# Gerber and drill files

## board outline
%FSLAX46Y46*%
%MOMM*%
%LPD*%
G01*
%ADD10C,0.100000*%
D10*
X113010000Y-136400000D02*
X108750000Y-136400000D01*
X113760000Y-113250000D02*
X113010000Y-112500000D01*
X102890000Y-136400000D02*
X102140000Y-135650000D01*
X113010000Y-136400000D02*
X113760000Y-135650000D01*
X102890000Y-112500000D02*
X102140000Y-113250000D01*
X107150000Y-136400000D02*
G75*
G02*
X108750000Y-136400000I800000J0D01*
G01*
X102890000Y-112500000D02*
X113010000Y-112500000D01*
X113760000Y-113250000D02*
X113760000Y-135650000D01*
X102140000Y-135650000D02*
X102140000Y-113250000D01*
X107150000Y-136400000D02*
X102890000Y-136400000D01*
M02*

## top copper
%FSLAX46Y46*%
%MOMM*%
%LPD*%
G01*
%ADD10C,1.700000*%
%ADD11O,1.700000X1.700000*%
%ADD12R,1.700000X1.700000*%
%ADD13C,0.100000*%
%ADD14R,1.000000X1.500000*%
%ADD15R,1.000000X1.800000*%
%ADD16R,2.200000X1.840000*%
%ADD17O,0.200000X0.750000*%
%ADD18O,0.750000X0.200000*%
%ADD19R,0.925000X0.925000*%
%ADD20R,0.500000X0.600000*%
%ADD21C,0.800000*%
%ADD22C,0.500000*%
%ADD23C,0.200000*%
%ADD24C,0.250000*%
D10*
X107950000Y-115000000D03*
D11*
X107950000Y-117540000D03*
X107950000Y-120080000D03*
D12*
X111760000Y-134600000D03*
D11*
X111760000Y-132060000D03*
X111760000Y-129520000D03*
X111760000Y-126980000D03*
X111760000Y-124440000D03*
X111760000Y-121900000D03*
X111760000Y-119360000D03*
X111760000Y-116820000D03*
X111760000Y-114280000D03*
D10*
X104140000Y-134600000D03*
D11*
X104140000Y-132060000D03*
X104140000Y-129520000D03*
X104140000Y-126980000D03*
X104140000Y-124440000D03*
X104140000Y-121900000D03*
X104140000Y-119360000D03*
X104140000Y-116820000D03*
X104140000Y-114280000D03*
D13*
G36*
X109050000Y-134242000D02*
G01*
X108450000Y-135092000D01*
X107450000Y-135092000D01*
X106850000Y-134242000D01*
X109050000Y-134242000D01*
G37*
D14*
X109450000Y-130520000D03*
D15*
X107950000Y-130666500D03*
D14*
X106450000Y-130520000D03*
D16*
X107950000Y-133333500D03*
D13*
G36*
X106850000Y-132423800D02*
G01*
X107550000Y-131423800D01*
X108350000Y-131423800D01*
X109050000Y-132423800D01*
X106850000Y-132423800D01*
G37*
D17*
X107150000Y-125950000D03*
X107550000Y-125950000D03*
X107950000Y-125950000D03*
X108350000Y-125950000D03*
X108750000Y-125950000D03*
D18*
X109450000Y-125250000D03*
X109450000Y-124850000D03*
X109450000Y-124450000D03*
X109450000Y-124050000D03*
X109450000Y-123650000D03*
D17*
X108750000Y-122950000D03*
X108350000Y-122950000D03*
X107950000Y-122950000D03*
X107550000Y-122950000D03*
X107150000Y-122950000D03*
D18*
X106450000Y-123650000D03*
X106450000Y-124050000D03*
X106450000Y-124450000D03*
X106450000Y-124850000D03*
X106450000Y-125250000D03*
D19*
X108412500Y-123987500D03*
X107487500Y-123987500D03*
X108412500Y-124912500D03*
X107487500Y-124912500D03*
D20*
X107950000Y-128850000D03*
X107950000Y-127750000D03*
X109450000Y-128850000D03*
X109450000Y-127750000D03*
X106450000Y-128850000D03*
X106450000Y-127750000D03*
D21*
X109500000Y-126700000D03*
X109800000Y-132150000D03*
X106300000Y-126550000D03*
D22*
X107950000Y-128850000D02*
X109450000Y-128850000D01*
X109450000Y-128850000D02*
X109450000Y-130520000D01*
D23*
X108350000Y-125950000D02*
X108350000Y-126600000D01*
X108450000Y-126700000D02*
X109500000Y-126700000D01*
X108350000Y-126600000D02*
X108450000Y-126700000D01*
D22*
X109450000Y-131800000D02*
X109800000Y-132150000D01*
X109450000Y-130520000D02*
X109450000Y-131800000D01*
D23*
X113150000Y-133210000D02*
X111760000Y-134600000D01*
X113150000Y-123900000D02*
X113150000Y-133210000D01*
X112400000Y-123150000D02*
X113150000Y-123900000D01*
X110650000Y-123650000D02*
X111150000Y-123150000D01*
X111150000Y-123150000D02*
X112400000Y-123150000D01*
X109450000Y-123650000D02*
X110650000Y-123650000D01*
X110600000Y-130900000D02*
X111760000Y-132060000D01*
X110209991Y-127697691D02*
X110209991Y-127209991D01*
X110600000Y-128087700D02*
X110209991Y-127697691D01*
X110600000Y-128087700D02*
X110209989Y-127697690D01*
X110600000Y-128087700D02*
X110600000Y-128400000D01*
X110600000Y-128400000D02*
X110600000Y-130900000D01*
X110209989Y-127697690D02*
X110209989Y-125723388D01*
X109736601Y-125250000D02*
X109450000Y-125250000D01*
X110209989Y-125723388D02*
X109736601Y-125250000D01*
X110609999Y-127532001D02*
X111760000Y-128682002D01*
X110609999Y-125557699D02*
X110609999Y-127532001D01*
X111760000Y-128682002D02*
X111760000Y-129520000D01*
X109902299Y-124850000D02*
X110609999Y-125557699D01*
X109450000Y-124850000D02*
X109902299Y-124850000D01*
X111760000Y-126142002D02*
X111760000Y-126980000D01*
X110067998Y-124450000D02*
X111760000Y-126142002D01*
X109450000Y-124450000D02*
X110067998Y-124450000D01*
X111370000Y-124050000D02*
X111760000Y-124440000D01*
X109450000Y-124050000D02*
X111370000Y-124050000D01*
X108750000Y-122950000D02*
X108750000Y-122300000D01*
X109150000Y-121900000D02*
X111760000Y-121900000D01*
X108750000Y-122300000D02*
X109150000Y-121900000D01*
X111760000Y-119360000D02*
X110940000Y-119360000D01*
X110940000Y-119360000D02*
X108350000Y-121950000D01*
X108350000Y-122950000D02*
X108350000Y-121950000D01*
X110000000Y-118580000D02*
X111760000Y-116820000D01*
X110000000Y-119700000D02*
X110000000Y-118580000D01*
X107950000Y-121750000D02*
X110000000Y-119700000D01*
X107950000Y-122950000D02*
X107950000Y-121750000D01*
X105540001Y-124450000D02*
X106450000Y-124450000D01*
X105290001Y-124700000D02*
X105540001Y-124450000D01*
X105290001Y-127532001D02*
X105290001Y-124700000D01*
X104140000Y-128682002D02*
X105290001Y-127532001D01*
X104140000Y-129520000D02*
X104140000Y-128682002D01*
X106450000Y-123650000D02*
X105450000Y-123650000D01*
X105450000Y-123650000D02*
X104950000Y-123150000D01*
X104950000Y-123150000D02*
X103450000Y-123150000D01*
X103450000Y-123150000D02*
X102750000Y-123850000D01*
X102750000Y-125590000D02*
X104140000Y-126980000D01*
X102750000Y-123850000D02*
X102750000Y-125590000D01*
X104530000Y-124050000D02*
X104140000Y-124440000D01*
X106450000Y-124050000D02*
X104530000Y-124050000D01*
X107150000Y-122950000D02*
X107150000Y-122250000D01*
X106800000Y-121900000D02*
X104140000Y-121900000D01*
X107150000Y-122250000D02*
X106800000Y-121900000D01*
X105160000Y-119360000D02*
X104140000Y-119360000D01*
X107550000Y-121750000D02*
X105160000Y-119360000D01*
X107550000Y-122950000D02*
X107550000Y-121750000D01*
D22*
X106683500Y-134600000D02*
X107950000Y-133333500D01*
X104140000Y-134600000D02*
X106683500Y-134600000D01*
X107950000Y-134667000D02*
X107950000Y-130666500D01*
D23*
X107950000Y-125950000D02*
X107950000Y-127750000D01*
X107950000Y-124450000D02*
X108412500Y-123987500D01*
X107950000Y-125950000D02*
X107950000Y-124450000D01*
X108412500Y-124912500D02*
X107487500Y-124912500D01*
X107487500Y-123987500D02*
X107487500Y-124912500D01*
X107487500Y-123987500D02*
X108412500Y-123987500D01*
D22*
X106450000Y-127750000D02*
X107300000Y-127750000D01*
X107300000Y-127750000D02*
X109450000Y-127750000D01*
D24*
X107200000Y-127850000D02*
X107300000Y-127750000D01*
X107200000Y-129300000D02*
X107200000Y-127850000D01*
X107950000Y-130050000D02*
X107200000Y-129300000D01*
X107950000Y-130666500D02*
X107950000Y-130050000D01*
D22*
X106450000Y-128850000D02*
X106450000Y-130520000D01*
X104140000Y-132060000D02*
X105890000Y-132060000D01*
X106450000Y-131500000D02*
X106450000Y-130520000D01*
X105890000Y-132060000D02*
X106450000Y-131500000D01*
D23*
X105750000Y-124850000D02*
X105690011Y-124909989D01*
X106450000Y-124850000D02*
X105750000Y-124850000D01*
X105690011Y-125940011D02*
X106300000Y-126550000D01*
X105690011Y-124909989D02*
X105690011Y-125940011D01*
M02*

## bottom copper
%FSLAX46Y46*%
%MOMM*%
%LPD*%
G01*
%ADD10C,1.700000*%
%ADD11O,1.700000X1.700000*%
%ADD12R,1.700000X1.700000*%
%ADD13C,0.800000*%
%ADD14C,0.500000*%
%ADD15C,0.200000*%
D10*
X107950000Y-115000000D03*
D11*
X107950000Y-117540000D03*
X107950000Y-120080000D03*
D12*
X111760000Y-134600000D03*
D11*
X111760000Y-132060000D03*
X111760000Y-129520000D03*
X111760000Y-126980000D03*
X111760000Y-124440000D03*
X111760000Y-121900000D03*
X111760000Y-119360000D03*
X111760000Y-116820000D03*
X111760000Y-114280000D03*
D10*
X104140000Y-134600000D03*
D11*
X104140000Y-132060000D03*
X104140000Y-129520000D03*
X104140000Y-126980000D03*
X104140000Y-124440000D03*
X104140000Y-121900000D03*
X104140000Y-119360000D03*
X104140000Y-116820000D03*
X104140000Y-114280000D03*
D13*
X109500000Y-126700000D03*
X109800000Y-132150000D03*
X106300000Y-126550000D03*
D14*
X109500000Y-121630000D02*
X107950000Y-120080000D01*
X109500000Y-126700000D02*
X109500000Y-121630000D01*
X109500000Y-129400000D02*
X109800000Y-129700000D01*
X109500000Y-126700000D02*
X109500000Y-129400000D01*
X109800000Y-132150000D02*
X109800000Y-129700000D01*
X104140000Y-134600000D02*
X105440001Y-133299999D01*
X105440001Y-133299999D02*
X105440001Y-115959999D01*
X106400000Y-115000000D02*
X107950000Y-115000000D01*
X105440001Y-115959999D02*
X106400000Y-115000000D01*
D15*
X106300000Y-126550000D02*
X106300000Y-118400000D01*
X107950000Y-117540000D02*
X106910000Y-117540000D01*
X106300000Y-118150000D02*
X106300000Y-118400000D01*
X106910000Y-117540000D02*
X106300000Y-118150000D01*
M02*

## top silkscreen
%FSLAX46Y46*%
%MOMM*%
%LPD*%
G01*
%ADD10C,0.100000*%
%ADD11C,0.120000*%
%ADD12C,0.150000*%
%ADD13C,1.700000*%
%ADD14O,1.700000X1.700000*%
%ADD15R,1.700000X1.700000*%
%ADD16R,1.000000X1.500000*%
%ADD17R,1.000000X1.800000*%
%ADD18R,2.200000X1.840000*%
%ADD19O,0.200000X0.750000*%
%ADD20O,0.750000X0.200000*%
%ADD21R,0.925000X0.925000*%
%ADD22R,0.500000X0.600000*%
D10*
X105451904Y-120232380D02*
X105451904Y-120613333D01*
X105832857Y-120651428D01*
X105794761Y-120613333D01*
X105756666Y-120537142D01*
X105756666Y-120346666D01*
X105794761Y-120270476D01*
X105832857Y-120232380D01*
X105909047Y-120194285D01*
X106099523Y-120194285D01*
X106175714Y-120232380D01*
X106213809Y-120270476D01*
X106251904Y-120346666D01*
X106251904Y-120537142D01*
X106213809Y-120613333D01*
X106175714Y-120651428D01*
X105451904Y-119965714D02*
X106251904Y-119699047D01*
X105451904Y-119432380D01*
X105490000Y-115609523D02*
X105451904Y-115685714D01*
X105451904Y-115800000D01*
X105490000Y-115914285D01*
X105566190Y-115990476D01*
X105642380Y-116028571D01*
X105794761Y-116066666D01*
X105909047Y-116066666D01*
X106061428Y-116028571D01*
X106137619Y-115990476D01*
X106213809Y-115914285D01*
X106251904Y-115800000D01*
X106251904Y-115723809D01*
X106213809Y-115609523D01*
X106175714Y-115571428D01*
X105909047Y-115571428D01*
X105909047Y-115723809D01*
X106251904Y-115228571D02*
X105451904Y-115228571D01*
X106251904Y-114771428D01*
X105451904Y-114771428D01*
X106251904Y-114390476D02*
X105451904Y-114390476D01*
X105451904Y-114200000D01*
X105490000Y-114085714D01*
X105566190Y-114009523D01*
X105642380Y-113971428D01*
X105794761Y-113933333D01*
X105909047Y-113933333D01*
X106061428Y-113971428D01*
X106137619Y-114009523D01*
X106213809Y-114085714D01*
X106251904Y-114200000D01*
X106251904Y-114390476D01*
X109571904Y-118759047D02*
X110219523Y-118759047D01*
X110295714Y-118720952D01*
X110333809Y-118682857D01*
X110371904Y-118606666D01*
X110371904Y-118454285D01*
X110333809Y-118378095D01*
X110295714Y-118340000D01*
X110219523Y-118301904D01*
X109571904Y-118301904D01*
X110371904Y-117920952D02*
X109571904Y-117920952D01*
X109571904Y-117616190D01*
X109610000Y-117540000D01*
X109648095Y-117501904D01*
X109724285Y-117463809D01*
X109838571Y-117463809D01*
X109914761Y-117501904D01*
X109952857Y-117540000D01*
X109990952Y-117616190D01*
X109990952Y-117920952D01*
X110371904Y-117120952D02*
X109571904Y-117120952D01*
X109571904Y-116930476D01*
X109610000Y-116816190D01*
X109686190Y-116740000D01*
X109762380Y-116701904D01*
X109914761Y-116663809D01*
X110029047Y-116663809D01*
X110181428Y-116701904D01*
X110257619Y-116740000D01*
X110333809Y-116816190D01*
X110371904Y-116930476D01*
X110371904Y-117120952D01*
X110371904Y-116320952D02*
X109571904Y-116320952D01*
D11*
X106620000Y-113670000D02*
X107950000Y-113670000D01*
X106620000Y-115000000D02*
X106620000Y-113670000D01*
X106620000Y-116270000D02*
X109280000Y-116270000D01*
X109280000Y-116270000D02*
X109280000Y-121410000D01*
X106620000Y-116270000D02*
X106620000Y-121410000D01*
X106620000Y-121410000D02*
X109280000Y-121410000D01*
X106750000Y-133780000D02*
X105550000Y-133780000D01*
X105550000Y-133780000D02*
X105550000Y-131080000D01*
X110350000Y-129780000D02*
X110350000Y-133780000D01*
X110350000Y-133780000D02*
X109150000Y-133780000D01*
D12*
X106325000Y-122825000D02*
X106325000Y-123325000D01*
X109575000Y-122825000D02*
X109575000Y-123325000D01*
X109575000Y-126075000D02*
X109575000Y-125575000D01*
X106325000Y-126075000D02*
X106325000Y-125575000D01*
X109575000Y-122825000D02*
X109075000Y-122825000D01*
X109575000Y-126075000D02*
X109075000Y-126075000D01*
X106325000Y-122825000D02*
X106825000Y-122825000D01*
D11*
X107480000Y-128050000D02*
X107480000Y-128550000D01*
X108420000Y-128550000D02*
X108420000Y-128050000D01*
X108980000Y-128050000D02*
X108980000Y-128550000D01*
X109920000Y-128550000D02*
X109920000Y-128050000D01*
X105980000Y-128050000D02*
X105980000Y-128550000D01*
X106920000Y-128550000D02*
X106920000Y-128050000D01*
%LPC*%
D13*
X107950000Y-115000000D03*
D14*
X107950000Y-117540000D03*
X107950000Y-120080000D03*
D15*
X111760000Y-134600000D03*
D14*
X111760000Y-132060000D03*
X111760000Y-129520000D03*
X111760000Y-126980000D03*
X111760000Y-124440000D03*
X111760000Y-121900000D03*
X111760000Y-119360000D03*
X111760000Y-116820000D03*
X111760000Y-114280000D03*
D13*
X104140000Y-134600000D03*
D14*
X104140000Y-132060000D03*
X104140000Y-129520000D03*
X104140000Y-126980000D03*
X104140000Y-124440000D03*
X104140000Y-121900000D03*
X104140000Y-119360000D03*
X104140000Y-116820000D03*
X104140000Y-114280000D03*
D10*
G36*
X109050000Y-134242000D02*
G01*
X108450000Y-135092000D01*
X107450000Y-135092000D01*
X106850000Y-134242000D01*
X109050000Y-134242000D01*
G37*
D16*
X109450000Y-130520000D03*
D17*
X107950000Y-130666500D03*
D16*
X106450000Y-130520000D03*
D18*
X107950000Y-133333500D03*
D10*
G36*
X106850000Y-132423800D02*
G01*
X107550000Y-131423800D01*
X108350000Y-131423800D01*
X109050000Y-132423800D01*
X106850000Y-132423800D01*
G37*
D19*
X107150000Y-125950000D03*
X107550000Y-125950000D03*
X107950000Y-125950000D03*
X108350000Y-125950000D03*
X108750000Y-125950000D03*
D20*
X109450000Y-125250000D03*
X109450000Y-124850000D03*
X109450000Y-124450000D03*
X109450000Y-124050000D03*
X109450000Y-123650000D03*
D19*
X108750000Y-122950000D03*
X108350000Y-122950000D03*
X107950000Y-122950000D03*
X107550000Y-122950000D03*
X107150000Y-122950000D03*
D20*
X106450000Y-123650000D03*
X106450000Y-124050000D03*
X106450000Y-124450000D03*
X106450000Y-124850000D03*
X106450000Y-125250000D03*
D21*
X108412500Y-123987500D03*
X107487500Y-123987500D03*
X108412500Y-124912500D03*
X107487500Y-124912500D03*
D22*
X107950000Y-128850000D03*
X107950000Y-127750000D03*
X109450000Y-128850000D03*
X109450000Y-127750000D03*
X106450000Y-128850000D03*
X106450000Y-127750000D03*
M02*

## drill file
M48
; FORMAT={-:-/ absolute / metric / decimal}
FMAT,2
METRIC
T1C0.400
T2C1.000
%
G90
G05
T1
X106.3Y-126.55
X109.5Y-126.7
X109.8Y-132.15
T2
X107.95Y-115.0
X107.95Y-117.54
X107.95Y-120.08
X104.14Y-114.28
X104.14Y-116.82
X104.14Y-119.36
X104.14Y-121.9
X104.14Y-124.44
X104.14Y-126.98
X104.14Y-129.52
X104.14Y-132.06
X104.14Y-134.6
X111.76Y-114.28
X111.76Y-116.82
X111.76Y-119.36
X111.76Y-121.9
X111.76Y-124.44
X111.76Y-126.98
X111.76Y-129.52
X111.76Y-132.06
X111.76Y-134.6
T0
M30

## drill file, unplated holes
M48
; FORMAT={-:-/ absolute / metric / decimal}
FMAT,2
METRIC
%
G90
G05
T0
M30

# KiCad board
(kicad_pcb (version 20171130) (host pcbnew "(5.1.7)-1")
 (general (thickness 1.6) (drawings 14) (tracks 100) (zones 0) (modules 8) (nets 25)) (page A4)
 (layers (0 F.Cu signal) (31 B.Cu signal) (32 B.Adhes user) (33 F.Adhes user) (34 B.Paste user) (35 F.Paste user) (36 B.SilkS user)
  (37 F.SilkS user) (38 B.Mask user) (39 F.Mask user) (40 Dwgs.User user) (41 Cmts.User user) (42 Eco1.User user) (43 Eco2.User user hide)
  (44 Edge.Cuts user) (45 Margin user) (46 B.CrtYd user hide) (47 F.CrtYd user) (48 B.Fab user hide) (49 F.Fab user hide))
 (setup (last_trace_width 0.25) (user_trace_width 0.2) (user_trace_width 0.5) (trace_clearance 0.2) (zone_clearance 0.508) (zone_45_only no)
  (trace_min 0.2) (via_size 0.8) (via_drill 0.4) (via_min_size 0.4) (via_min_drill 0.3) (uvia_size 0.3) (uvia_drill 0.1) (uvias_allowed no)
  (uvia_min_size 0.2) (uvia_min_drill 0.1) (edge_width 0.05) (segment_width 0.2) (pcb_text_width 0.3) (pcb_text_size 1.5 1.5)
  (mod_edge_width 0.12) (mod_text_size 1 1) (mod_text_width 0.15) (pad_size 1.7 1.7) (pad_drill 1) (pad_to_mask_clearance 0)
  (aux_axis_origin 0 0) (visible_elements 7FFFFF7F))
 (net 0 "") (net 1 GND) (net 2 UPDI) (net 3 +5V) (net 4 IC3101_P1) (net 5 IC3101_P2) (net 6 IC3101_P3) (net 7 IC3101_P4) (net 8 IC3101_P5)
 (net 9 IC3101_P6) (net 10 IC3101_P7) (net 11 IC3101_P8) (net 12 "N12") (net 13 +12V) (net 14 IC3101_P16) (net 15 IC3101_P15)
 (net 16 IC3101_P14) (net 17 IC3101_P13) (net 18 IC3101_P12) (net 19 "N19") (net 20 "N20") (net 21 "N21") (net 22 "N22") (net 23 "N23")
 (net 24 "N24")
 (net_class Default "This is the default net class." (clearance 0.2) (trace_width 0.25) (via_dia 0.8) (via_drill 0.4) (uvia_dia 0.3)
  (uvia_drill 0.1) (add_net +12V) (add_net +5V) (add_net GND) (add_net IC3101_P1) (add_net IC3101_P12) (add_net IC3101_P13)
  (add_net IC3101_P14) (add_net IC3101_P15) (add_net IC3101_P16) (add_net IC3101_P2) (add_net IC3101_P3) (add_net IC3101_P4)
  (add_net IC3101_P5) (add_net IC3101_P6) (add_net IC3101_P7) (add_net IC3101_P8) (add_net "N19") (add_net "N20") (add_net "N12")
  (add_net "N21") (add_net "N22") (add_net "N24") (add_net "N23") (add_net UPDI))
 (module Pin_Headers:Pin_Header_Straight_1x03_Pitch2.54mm (layer F.Cu) (at 107.95 115)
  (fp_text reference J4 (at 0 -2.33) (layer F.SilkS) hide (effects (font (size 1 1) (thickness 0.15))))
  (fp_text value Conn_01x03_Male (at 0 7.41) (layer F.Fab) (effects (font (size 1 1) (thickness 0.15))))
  (fp_line (start -1.33 -1.33) (end 0 -1.33) (layer F.SilkS) (width 0.12))
  (fp_line (start -1.33 0) (end -1.33 -1.33) (layer F.SilkS) (width 0.12))
  (fp_line (start -1.33 1.27) (end 1.33 1.27) (layer F.SilkS) (width 0.12))
  (fp_line (start 1.33 1.27) (end 1.33 6.41) (layer F.SilkS) (width 0.12))
  (fp_line (start -1.33 1.27) (end -1.33 6.41) (layer F.SilkS) (width 0.12))
  (fp_line (start -1.33 6.41) (end 1.33 6.41) (layer F.SilkS) (width 0.12))
  (pad 1 thru_hole circle (at 0 0) (size 1.7 1.7) (drill 1) (layers *.Cu *.Mask) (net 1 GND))
  (pad 2 thru_hole oval (at 0 2.54) (size 1.7 1.7) (drill 1) (layers *.Cu *.Mask) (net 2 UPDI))
  (pad 3 thru_hole oval (at 0 5.08) (size 1.7 1.7) (drill 1) (layers *.Cu *.Mask) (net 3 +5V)))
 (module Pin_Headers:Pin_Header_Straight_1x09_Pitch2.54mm (layer B.Cu) (at 111.76 134.6)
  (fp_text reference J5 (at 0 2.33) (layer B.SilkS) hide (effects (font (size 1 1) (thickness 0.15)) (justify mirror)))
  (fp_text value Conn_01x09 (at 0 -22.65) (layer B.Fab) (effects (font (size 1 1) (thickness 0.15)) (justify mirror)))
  (pad 1 thru_hole rect (at 0 0) (size 1.7 1.7) (drill 1) (layers *.Cu *.Mask) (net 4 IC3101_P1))
  (pad 2 thru_hole oval (at 0 -2.54) (size 1.7 1.7) (drill 1) (layers *.Cu *.Mask) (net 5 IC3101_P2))
  (pad 3 thru_hole oval (at 0 -5.08) (size 1.7 1.7) (drill 1) (layers *.Cu *.Mask) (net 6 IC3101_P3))
  (pad 4 thru_hole oval (at 0 -7.62) (size 1.7 1.7) (drill 1) (layers *.Cu *.Mask) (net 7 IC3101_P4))
  (pad 5 thru_hole oval (at 0 -10.16) (size 1.7 1.7) (drill 1) (layers *.Cu *.Mask) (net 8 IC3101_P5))
  (pad 6 thru_hole oval (at 0 -12.7) (size 1.7 1.7) (drill 1) (layers *.Cu *.Mask) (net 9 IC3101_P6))
  (pad 7 thru_hole oval (at 0 -15.24) (size 1.7 1.7) (drill 1) (layers *.Cu *.Mask) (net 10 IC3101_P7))
  (pad 8 thru_hole oval (at 0 -17.78) (size 1.7 1.7) (drill 1) (layers *.Cu *.Mask) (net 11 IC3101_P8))
  (pad 9 thru_hole oval (at 0 -20.32) (size 1.7 1.7) (drill 1) (layers *.Cu *.Mask) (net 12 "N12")))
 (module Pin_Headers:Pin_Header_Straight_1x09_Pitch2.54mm (layer B.Cu) (at 104.14 134.6)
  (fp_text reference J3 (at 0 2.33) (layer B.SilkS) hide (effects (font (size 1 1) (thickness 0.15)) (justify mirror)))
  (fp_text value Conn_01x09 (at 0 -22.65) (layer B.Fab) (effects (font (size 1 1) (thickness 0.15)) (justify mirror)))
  (pad 1 thru_hole circle (at 0 0) (size 1.7 1.7) (drill 1) (layers *.Cu *.Mask) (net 1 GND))
  (pad 2 thru_hole oval (at 0 -2.54) (size 1.7 1.7) (drill 1) (layers *.Cu *.Mask) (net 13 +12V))
  (pad 3 thru_hole oval (at 0 -5.08) (size 1.7 1.7) (drill 1) (layers *.Cu *.Mask) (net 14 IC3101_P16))
  (pad 4 thru_hole oval (at 0 -7.62) (size 1.7 1.7) (drill 1) (layers *.Cu *.Mask) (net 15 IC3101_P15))
  (pad 5 thru_hole oval (at 0 -10.16) (size 1.7 1.7) (drill 1) (layers *.Cu *.Mask) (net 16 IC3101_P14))
  (pad 6 thru_hole oval (at 0 -12.7) (size 1.7 1.7) (drill 1) (layers *.Cu *.Mask) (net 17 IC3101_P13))
  (pad 7 thru_hole oval (at 0 -15.24) (size 1.7 1.7) (drill 1) (layers *.Cu *.Mask) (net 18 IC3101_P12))
  (pad 8 thru_hole oval (at 0 -17.78) (size 1.7 1.7) (drill 1) (layers *.Cu *.Mask) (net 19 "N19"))
  (pad 9 thru_hole oval (at 0 -20.32) (size 1.7 1.7) (drill 1) (layers *.Cu *.Mask) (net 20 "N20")))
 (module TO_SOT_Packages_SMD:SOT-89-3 (layer F.Cu) (at 107.95 132 270)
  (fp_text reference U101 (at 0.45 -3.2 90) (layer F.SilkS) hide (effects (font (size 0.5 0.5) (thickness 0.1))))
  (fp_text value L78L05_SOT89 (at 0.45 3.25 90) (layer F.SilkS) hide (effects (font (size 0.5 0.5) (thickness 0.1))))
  (fp_line (start 1.78 1.2) (end 1.78 2.4) (layer F.SilkS) (width 0.12))
  (fp_line (start 1.78 2.4) (end -0.92 2.4) (layer F.SilkS) (width 0.12))
  (fp_line (start -2.22 -2.4) (end 1.78 -2.4) (layer F.SilkS) (width 0.12))
  (fp_line (start 1.78 -2.4) (end 1.78 -1.2) (layer F.SilkS) (width 0.12))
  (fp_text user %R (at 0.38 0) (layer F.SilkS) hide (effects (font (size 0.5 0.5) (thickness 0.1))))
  (pad 2 smd trapezoid (at 2.667 0 180) (size 1.6 0.85) (rect_delta 0 0.6) (layers F.Cu F.Paste F.Mask) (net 1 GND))
  (pad 1 smd rect (at -1.48 -1.5 180) (size 1 1.5) (layers F.Cu F.Paste F.Mask) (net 3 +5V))
  (pad 2 smd rect (at -1.3335 0 180) (size 1 1.8) (layers F.Cu F.Paste F.Mask) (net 1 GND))
  (pad 3 smd rect (at -1.48 1.5 180) (size 1 1.5) (layers F.Cu F.Paste F.Mask) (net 13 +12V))
  (pad 2 smd rect (at 1.3335 0 180) (size 2.2 1.84) (layers F.Cu F.Paste F.Mask) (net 1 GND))
  (pad 2 smd trapezoid (at -0.0762 0) (size 1.5 1) (rect_delta 0 0.7) (layers F.Cu F.Paste F.Mask) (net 1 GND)))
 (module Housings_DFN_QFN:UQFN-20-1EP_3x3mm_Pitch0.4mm (layer F.Cu) (at 107.95 124.45 90)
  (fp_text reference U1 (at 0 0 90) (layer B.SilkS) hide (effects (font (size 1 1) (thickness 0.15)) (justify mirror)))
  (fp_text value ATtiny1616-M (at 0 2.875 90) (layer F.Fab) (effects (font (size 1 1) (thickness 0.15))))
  (fp_line (start 1.625 -1.625) (end 1.125 -1.625) (layer F.SilkS) (width 0.15))
  (fp_line (start 1.625 1.625) (end 1.125 1.625) (layer F.SilkS) (width 0.15))
  (fp_line (start -1.625 1.625) (end -1.125 1.625) (layer F.SilkS) (width 0.15))
  (fp_line (start -1.625 -1.625) (end -1.125 -1.625) (layer F.SilkS) (width 0.15))
  (fp_line (start 1.625 1.625) (end 1.625 1.125) (layer F.SilkS) (width 0.15))
  (fp_line (start -1.625 1.625) (end -1.625 1.125) (layer F.SilkS) (width 0.15))
  (fp_line (start 1.625 -1.625) (end 1.625 -1.125) (layer F.SilkS) (width 0.15))
  (pad 1 smd oval (at -1.5 -0.8 90) (size 0.75 0.2) (layers F.Cu F.Paste F.Mask) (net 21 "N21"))
  (pad 2 smd oval (at -1.5 -0.4 90) (size 0.75 0.2) (layers F.Cu F.Paste F.Mask) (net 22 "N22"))
  (pad 3 smd oval (at -1.5 0 90) (size 0.75 0.2) (layers F.Cu F.Paste F.Mask) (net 1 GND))
  (pad 4 smd oval (at -1.5 0.4 90) (size 0.75 0.2) (layers F.Cu F.Paste F.Mask) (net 3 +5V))
  (pad 5 smd oval (at -1.5 0.8 90) (size 0.75 0.2) (layers F.Cu F.Paste F.Mask) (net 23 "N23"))
  (pad 6 smd oval (at -0.8 1.5 180) (size 0.75 0.2) (layers F.Cu F.Paste F.Mask) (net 5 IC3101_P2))
  (pad 7 smd oval (at -0.4 1.5 180) (size 0.75 0.2) (layers F.Cu F.Paste F.Mask) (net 6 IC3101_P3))
  (pad 8 smd oval (at 0 1.5 180) (size 0.75 0.2) (layers F.Cu F.Paste F.Mask) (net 7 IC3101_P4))
  (pad 9 smd oval (at 0.4 1.5 180) (size 0.75 0.2) (layers F.Cu F.Paste F.Mask) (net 8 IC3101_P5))
  (pad 10 smd oval (at 0.8 1.5 180) (size 0.75 0.2) (layers F.Cu F.Paste F.Mask) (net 4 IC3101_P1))
  (pad 11 smd oval (at 1.5 0.8 90) (size 0.75 0.2) (layers F.Cu F.Paste F.Mask) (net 9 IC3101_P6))
  (pad 12 smd oval (at 1.5 0.4 90) (size 0.75 0.2) (layers F.Cu F.Paste F.Mask) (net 10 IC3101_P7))
  (pad 13 smd oval (at 1.5 0 90) (size 0.75 0.2) (layers F.Cu F.Paste F.Mask) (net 11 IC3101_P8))
  (pad 14 smd oval (at 1.5 -0.4 90) (size 0.75 0.2) (layers F.Cu F.Paste F.Mask) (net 18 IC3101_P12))
  (pad 15 smd oval (at 1.5 -0.8 90) (size 0.75 0.2) (layers F.Cu F.Paste F.Mask) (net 17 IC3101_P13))
  (pad 16 smd oval (at 0.8 -1.5 180) (size 0.75 0.2) (layers F.Cu F.Paste F.Mask) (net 15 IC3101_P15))
  (pad 17 smd oval (at 0.4 -1.5 180) (size 0.75 0.2) (layers F.Cu F.Paste F.Mask) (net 16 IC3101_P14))
  (pad 18 smd oval (at 0 -1.5 180) (size 0.75 0.2) (layers F.Cu F.Paste F.Mask) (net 14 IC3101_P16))
  (pad 19 smd oval (at -0.4 -1.5 180) (size 0.75 0.2) (layers F.Cu F.Paste F.Mask) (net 2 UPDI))
  (pad 20 smd oval (at -0.8 -1.5 180) (size 0.75 0.2) (layers F.Cu F.Paste F.Mask) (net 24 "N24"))
  (pad 21 smd rect (at 0.4625 0.4625 90) (size 0.925 0.925) (layers F.Cu F.Paste F.Mask) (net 1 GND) (solder_paste_margin_ratio -0.2))
  (pad 21 smd rect (at 0.4625 -0.4625 90) (size 0.925 0.925) (layers F.Cu F.Paste F.Mask) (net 1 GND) (solder_paste_margin_ratio -0.2))
  (pad 21 smd rect (at -0.4625 0.4625 90) (size 0.925 0.925) (layers F.Cu F.Paste F.Mask) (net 1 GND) (solder_paste_margin_ratio -0.2))
  (pad 21 smd rect (at -0.4625 -0.4625 90) (size 0.925 0.925) (layers F.Cu F.Paste F.Mask) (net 1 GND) (solder_paste_margin_ratio -0.2)))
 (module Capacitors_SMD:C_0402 (layer F.Cu) (at 107.95 128.3 90)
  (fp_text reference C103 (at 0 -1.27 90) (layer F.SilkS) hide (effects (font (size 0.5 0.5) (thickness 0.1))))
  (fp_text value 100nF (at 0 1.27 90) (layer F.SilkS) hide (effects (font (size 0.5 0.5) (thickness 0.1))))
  (fp_line (start 0.25 -0.47) (end -0.25 -0.47) (layer F.SilkS) (width 0.12))
  (fp_line (start -0.25 0.47) (end 0.25 0.47) (layer F.SilkS) (width 0.12))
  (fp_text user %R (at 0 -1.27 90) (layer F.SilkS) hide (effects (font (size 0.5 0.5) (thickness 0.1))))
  (pad 1 smd rect (at -0.55 0 90) (size 0.6 0.5) (layers F.Cu F.Paste F.Mask) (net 3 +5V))
  (pad 2 smd rect (at 0.55 0 90) (size 0.6 0.5) (layers F.Cu F.Paste F.Mask) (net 1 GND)))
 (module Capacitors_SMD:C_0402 (layer F.Cu) (at 109.45 128.3 90)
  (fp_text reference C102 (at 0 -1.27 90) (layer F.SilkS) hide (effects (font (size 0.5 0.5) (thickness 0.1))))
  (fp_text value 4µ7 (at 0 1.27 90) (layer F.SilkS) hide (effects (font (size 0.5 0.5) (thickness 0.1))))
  (fp_line (start 0.25 -0.47) (end -0.25 -0.47) (layer F.SilkS) (width 0.12))
  (fp_line (start -0.25 0.47) (end 0.25 0.47) (layer F.SilkS) (width 0.12))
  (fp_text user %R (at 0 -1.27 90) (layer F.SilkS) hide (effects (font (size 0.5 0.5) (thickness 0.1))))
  (pad 1 smd rect (at -0.55 0 90) (size 0.6 0.5) (layers F.Cu F.Paste F.Mask) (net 3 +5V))
  (pad 2 smd rect (at 0.55 0 90) (size 0.6 0.5) (layers F.Cu F.Paste F.Mask) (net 1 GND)))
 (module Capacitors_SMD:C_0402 (layer F.Cu) (at 106.45 128.3 90)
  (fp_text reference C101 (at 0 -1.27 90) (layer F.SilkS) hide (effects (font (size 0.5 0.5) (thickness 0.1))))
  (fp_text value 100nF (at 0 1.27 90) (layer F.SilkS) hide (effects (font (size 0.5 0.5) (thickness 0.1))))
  (fp_line (start 0.25 -0.47) (end -0.25 -0.47) (layer F.SilkS) (width 0.12))
  (fp_line (start -0.25 0.47) (end 0.25 0.47) (layer F.SilkS) (width 0.12))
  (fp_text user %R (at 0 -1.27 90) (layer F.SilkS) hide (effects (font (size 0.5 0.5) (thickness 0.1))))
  (pad 1 smd rect (at -0.55 0 90) (size 0.6 0.5) (layers F.Cu F.Paste F.Mask) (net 13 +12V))
  (pad 2 smd rect (at 0.55 0 90) (size 0.6 0.5) (layers F.Cu F.Paste F.Mask) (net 1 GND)))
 (gr_line (start 113.01 136.4) (end 108.75 136.4) (layer Edge.Cuts) (width 0.1))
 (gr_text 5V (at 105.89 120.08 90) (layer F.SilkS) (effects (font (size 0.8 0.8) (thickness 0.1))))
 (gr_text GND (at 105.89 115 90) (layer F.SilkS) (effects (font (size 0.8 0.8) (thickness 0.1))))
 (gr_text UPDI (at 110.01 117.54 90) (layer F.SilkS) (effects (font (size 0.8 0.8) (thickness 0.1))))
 (gr_line (start 113.76 113.25) (end 113.01 112.5) (layer Edge.Cuts) (width 0.1))
 (gr_line (start 102.89 136.4) (end 102.14 135.65) (layer Edge.Cuts) (width 0.1))
 (gr_line (start 113.01 136.4) (end 113.76 135.65) (layer Edge.Cuts) (width 0.1))
 (gr_line (start 102.89 112.5) (end 102.14 113.25) (layer Edge.Cuts) (width 0.1))
 (gr_arc (start 107.95 136.4) (end 108.75 136.4) (angle -180) (layer Edge.Cuts) (width 0.1))
 (gr_line (start 102.89 112.5) (end 113.01 112.5) (layer Edge.Cuts) (width 0.1))
 (gr_line (start 113.76 113.25) (end 113.76 135.65) (layer Edge.Cuts) (width 0.1))
 (gr_line (start 102.14 135.65) (end 102.14 113.25) (layer Edge.Cuts) (width 0.1))
 (gr_line (start 107.15 136.4) (end 102.89 136.4) (layer Edge.Cuts) (width 0.1))
 (via (at 109.5 126.7) (size 0.8) (drill 0.4) (layers F.Cu B.Cu) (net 3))
 (segment (start 107.95 128.85) (end 109.45 128.85) (width 0.5) (layer F.Cu) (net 3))
 (segment (start 109.45 128.85) (end 109.45 130.52) (width 0.5) (layer F.Cu) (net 3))
 (segment (start 108.35 125.95) (end 108.35 126.6) (width 0.2) (layer F.Cu) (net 3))
 (segment (start 108.45 126.7) (end 109.5 126.7) (width 0.2) (layer F.Cu) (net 3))
 (segment (start 108.35 126.6) (end 108.45 126.7) (width 0.2) (layer F.Cu) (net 3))
 (via (at 109.8 132.15) (size 0.8) (drill 0.4) (layers F.Cu B.Cu) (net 3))
 (segment (start 109.45 131.8) (end 109.8 132.15) (width 0.5) (layer F.Cu) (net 3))
 (segment (start 109.45 130.52) (end 109.45 131.8) (width 0.5) (layer F.Cu) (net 3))
 (segment (start 109.5 121.63) (end 107.95 120.08) (width 0.5) (layer B.Cu) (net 3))
 (segment (start 109.5 126.7) (end 109.5 121.63) (width 0.5) (layer B.Cu) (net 3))
 (segment (start 109.5 129.4) (end 109.8 129.7) (width 0.5) (layer B.Cu) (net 3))
 (segment (start 109.5 126.7) (end 109.5 129.4) (width 0.5) (layer B.Cu) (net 3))
 (segment (start 109.8 132.15) (end 109.8 129.7) (width 0.5) (layer B.Cu) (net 3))
 (segment (start 113.15 133.21) (end 111.76 134.6) (width 0.2) (layer F.Cu) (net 4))
 (segment (start 113.15 123.9) (end 113.15 133.21) (width 0.2) (layer F.Cu) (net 4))
 (segment (start 112.4 123.15) (end 113.15 123.9) (width 0.2) (layer F.Cu) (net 4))
 (segment (start 110.65 123.65) (end 111.15 123.15) (width 0.2) (layer F.Cu) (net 4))
 (segment (start 111.15 123.15) (end 112.4 123.15) (width 0.2) (layer F.Cu) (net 4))
 (segment (start 109.45 123.65) (end 110.65 123.65) (width 0.2) (layer F.Cu) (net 4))
 (segment (start 110.6 130.9) (end 111.76 132.06) (width 0.2) (layer F.Cu) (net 5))
 (segment (start 110.209991 127.697691) (end 110.209991 127.209991) (width 0.2) (layer F.Cu) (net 5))
 (segment (start 110.6 128.0877) (end 110.209991 127.697691) (width 0.2) (layer F.Cu) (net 5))
 (segment (start 110.6 128.0877) (end 110.209989 127.69769) (width 0.2) (layer F.Cu) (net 5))
 (segment (start 110.6 128.0877) (end 110.6 128.4) (width 0.2) (layer F.Cu) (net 5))
 (segment (start 110.6 128.4) (end 110.6 130.9) (width 0.2) (layer F.Cu) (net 5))
 (segment (start 110.209989 127.69769) (end 110.209989 125.723388) (width 0.2) (layer F.Cu) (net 5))
 (segment (start 109.736601 125.25) (end 109.45 125.25) (width 0.2) (layer F.Cu) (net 5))
 (segment (start 110.209989 125.723388) (end 109.736601 125.25) (width 0.2) (layer F.Cu) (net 5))
 (segment (start 110.609999 127.532001) (end 111.76 128.682002) (width 0.2) (layer F.Cu) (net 6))
 (segment (start 110.609999 125.557699) (end 110.609999 127.532001) (width 0.2) (layer F.Cu) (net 6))
 (segment (start 111.76 128.682002) (end 111.76 129.52) (width 0.2) (layer F.Cu) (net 6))
 (segment (start 109.902299 124.85) (end 110.609999 125.557699) (width 0.2) (layer F.Cu) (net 6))
 (segment (start 109.45 124.85) (end 109.902299 124.85) (width 0.2) (layer F.Cu) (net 6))
 (segment (start 111.76 126.142002) (end 111.76 126.98) (width 0.2) (layer F.Cu) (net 7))
 (segment (start 110.067998 124.45) (end 111.76 126.142002) (width 0.2) (layer F.Cu) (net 7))
 (segment (start 109.45 124.45) (end 110.067998 124.45) (width 0.2) (layer F.Cu) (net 7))
 (segment (start 111.37 124.05) (end 111.76 124.44) (width 0.2) (layer F.Cu) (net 8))
 (segment (start 109.45 124.05) (end 111.37 124.05) (width 0.2) (layer F.Cu) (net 8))
 (segment (start 108.75 122.95) (end 108.75 122.3) (width 0.2) (layer F.Cu) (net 9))
 (segment (start 109.15 121.9) (end 111.76 121.9) (width 0.2) (layer F.Cu) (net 9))
 (segment (start 108.75 122.3) (end 109.15 121.9) (width 0.2) (layer F.Cu) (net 9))
 (segment (start 111.76 119.36) (end 110.94 119.36) (width 0.2) (layer F.Cu) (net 10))
 (segment (start 110.94 119.36) (end 108.35 121.95) (width 0.2) (layer F.Cu) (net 10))
 (segment (start 108.35 122.95) (end 108.35 121.95) (width 0.2) (layer F.Cu) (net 10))
 (segment (start 110 118.58) (end 111.76 116.82) (width 0.2) (layer F.Cu) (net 11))
 (segment (start 110 119.7) (end 110 118.58) (width 0.2) (layer F.Cu) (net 11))
 (segment (start 107.95 121.75) (end 110 119.7) (width 0.2) (layer F.Cu) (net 11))
 (segment (start 107.95 122.95) (end 107.95 121.75) (width 0.2) (layer F.Cu) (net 11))
 (segment (start 105.540001 124.45) (end 106.45 124.45) (width 0.2) (layer F.Cu) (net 14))
 (segment (start 105.290001 124.7) (end 105.540001 124.45) (width 0.2) (layer F.Cu) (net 14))
 (segment (start 105.290001 127.532001) (end 105.290001 124.7) (width 0.2) (layer F.Cu) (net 14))
 (segment (start 104.14 128.682002) (end 105.290001 127.532001) (width 0.2) (layer F.Cu) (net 14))
 (segment (start 104.14 129.52) (end 104.14 128.682002) (width 0.2) (layer F.Cu) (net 14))
 (segment (start 106.45 123.65) (end 105.45 123.65) (width 0.2) (layer F.Cu) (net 15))
 (segment (start 105.45 123.65) (end 104.95 123.15) (width 0.2) (layer F.Cu) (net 15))
 (segment (start 104.95 123.15) (end 103.45 123.15) (width 0.2) (layer F.Cu) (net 15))
 (segment (start 103.45 123.15) (end 102.75 123.85) (width 0.2) (layer F.Cu) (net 15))
 (segment (start 102.75 125.59) (end 104.14 126.98) (width 0.2) (layer F.Cu) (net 15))
 (segment (start 102.75 123.85) (end 102.75 125.59) (width 0.2) (layer F.Cu) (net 15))
 (segment (start 104.53 124.05) (end 104.14 124.44) (width 0.2) (layer F.Cu) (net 16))
 (segment (start 106.45 124.05) (end 104.53 124.05) (width 0.2) (layer F.Cu) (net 16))
 (segment (start 107.15 122.95) (end 107.15 122.25) (width 0.2) (layer F.Cu) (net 17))
 (segment (start 106.8 121.9) (end 104.14 121.9) (width 0.2) (layer F.Cu) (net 17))
 (segment (start 107.15 122.25) (end 106.8 121.9) (width 0.2) (layer F.Cu) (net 17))
 (segment (start 105.16 119.36) (end 104.14 119.36) (width 0.2) (layer F.Cu) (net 18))
 (segment (start 107.55 121.75) (end 105.16 119.36) (width 0.2) (layer F.Cu) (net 18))
 (segment (start 107.55 122.95) (end 107.55 121.75) (width 0.2) (layer F.Cu) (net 18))
 (segment (start 106.6835 134.6) (end 107.95 133.3335) (width 0.5) (layer F.Cu) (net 1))
 (segment (start 104.14 134.6) (end 106.6835 134.6) (width 0.5) (layer F.Cu) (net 1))
 (segment (start 107.95 134.667) (end 107.95 130.6665) (width 0.5) (layer F.Cu) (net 1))
 (segment (start 107.95 125.95) (end 107.95 127.75) (width 0.2) (layer F.Cu) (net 1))
 (segment (start 107.95 124.45) (end 108.4125 123.9875) (width 0.2) (layer F.Cu) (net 1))
 (segment (start 107.95 125.95) (end 107.95 124.45) (width 0.2) (layer F.Cu) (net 1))
 (segment (start 108.4125 124.9125) (end 107.4875 124.9125) (width 0.2) (layer F.Cu) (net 1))
 (segment (start 107.4875 123.9875) (end 107.4875 124.9125) (width 0.2) (layer F.Cu) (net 1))
 (segment (start 107.4875 123.9875) (end 108.4125 123.9875) (width 0.2) (layer F.Cu) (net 1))
 (segment (start 106.45 127.75) (end 107.3 127.75) (width 0.5) (layer F.Cu) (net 1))
 (segment (start 107.3 127.75) (end 109.45 127.75) (width 0.5) (layer F.Cu) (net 1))
 (segment (start 107.2 127.85) (end 107.3 127.75) (width 0.25) (layer F.Cu) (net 1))
 (segment (start 107.2 129.3) (end 107.2 127.85) (width 0.25) (layer F.Cu) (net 1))
 (segment (start 107.95 130.05) (end 107.2 129.3) (width 0.25) (layer F.Cu) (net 1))
 (segment (start 107.95 130.6665) (end 107.95 130.05) (width 0.25) (layer F.Cu) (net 1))
 (segment (start 104.14 134.6) (end 105.440001 133.299999) (width 0.5) (layer B.Cu) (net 1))
 (segment (start 105.440001 133.299999) (end 105.440001 115.959999) (width 0.5) (layer B.Cu) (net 1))
 (segment (start 106.4 115) (end 107.95 115) (width 0.5) (layer B.Cu) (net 1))
 (segment (start 105.440001 115.959999) (end 106.4 115) (width 0.5) (layer B.Cu) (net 1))
 (segment (start 106.45 128.85) (end 106.45 130.52) (width 0.5) (layer F.Cu) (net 13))
 (segment (start 104.14 132.06) (end 105.89 132.06) (width 0.5) (layer F.Cu) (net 13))
 (segment (start 106.45 131.5) (end 106.45 130.52) (width 0.5) (layer F.Cu) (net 13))
 (segment (start 105.89 132.06) (end 106.45 131.5) (width 0.5) (layer F.Cu) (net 13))
 (segment (start 105.75 124.85) (end 105.690011 124.909989) (width 0.2) (layer F.Cu) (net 2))
 (segment (start 106.45 124.85) (end 105.75 124.85) (width 0.2) (layer F.Cu) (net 2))
 (via (at 106.3 126.55) (size 0.8) (drill 0.4) (layers F.Cu B.Cu) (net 2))
 (segment (start 105.690011 125.940011) (end 106.3 126.55) (width 0.2) (layer F.Cu) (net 2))
 (segment (start 105.690011 124.909989) (end 105.690011 125.940011) (width 0.2) (layer F.Cu) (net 2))
 (segment (start 106.3 126.55) (end 106.3 118.4) (width 0.2) (layer B.Cu) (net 2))
 (segment (start 107.95 117.54) (end 106.91 117.54) (width 0.2) (layer B.Cu) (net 2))
 (segment (start 106.3 118.15) (end 106.3 118.4) (width 0.2) (layer B.Cu) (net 2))
 (segment (start 106.91 117.54) (end 106.3 118.15) (width 0.2) (layer B.Cu) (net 2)))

